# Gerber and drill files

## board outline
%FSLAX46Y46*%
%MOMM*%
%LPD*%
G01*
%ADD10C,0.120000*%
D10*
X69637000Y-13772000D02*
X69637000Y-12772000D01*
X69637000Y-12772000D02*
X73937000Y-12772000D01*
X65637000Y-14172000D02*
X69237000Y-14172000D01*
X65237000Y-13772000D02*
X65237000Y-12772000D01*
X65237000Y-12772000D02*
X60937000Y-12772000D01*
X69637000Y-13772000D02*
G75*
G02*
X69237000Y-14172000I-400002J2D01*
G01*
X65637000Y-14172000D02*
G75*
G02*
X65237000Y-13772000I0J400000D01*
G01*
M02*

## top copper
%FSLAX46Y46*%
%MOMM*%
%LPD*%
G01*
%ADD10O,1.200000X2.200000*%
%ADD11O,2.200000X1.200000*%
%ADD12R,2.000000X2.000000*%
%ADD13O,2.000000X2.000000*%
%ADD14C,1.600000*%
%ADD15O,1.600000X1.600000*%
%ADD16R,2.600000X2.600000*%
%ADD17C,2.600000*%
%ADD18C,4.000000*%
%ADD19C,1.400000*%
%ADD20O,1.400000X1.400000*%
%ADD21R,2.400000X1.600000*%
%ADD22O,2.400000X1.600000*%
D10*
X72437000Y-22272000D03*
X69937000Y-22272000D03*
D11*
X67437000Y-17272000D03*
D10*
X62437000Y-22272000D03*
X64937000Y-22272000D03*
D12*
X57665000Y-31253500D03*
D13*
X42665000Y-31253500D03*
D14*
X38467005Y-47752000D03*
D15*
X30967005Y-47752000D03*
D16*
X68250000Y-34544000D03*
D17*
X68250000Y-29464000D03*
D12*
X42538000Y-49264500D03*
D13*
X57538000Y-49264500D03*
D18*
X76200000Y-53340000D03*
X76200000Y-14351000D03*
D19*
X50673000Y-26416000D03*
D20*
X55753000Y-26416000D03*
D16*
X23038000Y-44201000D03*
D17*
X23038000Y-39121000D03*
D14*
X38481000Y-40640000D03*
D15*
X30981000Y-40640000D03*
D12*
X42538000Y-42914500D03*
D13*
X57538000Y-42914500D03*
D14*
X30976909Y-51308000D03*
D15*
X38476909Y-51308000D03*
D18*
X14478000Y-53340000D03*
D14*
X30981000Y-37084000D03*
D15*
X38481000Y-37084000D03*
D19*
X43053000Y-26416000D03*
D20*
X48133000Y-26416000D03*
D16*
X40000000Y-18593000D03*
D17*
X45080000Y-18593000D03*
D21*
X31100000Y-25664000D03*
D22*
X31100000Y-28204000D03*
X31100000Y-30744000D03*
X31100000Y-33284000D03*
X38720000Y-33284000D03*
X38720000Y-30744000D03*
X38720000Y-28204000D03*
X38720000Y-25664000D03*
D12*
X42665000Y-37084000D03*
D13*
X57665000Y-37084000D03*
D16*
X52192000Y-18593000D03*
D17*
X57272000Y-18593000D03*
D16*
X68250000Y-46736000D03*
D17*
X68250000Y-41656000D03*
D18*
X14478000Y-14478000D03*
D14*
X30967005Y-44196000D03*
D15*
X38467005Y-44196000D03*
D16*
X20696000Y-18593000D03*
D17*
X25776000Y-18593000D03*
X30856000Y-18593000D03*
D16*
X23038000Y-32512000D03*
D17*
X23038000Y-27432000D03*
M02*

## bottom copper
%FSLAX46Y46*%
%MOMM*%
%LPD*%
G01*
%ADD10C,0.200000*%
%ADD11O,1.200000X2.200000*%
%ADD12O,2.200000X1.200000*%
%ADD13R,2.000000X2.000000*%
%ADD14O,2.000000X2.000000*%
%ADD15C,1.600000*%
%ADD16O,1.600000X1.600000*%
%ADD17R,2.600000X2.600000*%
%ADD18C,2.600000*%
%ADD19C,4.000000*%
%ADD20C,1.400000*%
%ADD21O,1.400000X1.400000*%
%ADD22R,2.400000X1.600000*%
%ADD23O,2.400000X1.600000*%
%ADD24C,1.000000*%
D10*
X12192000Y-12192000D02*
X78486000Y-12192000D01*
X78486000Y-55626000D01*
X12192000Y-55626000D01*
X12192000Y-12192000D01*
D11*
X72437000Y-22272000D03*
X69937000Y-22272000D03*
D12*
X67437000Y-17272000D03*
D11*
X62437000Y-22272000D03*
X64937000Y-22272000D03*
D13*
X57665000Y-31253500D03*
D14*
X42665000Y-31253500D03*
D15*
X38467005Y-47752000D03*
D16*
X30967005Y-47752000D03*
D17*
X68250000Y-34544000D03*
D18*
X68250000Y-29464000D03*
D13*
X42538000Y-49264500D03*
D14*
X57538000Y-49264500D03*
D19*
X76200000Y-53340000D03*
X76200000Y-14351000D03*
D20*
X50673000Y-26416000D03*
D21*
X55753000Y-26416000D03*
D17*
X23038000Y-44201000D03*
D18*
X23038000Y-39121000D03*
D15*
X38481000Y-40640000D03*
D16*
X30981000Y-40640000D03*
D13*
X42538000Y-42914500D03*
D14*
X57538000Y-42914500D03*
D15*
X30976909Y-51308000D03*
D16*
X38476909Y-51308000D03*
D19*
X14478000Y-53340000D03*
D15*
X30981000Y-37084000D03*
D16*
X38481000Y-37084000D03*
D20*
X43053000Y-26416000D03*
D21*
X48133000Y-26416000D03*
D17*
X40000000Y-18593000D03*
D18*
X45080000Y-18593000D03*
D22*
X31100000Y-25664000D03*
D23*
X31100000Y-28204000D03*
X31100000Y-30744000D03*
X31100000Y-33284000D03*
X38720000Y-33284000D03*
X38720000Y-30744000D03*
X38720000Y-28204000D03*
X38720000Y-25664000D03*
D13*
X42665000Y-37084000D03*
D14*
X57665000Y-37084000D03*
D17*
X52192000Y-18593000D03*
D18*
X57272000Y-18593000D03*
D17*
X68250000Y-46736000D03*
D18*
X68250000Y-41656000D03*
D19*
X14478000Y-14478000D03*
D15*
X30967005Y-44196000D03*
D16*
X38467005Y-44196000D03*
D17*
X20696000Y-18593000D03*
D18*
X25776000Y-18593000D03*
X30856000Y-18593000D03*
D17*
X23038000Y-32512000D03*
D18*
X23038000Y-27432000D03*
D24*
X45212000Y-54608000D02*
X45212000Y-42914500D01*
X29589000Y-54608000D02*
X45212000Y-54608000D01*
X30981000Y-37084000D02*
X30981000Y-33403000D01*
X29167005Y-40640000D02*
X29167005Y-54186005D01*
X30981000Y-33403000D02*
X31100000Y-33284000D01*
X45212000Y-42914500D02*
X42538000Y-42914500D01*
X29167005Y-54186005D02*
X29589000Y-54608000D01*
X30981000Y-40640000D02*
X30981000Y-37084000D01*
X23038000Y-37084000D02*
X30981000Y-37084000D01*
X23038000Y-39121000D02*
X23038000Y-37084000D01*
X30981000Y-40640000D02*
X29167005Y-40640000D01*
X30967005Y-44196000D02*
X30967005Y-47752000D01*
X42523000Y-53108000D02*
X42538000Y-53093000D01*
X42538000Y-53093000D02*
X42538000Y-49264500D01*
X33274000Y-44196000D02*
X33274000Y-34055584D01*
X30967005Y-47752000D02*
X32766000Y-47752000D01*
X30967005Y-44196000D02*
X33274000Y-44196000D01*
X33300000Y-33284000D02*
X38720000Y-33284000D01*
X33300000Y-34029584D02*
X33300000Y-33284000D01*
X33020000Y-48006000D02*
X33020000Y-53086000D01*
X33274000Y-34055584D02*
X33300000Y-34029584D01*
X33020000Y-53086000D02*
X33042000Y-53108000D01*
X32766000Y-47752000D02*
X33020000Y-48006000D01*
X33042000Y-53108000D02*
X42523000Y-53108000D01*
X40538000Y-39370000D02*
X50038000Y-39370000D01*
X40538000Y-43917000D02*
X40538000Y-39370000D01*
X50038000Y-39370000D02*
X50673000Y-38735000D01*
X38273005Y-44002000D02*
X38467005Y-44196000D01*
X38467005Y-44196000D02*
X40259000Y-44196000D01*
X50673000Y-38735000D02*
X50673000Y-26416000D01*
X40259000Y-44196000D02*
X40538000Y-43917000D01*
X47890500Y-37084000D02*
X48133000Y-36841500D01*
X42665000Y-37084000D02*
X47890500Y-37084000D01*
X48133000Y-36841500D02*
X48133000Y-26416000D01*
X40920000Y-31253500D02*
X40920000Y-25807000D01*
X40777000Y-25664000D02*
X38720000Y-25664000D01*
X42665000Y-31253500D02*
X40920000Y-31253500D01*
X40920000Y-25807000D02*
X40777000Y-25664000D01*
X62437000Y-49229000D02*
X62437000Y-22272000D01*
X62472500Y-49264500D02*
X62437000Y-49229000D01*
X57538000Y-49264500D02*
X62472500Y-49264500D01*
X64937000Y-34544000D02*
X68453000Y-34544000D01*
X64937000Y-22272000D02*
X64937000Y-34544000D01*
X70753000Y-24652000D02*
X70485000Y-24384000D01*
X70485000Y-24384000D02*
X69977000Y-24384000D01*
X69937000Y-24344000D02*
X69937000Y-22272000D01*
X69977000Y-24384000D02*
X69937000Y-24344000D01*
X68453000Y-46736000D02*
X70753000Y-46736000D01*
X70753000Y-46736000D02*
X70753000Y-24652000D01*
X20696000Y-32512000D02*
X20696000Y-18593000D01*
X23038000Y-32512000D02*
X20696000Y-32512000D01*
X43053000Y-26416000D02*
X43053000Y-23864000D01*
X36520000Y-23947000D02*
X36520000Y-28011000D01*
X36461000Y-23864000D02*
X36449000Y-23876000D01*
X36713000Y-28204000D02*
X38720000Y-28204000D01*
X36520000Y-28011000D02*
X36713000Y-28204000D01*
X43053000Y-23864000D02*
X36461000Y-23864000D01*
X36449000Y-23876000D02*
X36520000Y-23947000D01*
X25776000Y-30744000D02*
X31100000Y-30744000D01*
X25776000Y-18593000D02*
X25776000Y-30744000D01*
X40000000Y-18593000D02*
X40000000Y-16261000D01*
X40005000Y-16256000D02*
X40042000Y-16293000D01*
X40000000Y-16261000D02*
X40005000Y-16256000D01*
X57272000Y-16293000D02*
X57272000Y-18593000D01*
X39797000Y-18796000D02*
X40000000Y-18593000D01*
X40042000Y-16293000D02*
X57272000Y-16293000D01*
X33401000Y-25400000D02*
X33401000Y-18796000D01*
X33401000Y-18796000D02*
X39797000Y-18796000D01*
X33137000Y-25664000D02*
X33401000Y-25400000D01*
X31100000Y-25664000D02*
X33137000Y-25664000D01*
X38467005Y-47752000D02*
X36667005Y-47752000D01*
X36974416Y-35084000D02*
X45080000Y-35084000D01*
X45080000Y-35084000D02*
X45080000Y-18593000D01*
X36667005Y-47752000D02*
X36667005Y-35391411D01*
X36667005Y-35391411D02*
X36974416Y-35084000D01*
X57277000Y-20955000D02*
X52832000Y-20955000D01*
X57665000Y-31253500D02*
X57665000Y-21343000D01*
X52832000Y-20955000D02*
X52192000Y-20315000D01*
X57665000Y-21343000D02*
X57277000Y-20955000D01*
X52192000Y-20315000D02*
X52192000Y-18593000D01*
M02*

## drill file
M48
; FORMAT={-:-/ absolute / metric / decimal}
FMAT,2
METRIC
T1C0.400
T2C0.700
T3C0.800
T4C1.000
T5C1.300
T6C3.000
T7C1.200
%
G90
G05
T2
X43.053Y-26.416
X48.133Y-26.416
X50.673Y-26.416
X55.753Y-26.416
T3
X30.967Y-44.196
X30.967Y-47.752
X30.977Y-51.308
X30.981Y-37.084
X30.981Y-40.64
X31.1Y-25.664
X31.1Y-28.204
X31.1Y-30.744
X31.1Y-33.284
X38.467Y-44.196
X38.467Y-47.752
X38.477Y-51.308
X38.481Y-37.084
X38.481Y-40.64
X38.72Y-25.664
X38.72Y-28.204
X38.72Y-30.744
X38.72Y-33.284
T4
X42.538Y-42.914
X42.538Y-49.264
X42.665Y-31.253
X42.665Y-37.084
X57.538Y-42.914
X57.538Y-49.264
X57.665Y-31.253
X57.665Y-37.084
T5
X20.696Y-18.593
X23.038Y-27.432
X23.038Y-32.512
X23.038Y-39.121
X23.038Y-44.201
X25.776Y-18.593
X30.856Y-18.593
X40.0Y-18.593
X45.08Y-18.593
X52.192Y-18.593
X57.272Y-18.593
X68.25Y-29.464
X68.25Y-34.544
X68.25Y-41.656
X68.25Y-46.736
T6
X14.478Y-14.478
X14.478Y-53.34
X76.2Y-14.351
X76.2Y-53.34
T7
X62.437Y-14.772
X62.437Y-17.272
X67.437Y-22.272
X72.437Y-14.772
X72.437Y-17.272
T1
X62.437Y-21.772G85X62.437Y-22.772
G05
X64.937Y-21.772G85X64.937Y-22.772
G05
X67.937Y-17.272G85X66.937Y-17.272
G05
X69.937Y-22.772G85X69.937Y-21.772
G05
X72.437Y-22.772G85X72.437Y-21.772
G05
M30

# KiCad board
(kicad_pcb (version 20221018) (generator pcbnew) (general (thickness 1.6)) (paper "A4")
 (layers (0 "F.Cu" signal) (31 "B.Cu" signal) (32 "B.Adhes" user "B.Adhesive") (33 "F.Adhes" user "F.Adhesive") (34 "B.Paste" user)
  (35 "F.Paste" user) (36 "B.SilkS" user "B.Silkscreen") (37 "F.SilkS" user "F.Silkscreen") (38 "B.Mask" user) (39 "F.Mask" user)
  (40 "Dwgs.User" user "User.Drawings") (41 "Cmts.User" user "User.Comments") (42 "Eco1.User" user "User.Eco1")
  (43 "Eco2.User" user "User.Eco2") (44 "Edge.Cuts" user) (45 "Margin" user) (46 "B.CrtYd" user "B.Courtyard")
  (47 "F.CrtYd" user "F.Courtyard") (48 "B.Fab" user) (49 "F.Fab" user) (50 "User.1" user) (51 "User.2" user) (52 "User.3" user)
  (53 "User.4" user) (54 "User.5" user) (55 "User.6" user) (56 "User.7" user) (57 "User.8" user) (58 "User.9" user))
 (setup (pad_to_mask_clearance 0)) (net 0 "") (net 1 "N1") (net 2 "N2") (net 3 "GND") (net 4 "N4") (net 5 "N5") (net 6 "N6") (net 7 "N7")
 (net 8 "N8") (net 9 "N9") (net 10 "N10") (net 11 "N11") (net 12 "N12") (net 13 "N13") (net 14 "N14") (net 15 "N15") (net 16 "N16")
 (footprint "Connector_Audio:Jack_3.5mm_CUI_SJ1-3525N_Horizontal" (layer "F.Cu") (at 67.437 17.272 180)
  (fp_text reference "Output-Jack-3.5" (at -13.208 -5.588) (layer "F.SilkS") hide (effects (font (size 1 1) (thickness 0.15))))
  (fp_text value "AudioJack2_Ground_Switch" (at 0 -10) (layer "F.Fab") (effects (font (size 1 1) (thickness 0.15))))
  (fp_line (start -2.2 3.5) (end -2.2 4.5) (stroke (width 0.12) (type solid)) (layer "Edge.Cuts"))
  (fp_line (start -2.2 4.5) (end -6.5 4.5) (stroke (width 0.12) (type solid)) (layer "Edge.Cuts"))
  (fp_line (start 1.8 3.1) (end -1.8 3.1) (stroke (width 0.12) (type solid)) (layer "Edge.Cuts"))
  (fp_line (start 2.2 3.5) (end 2.2 4.5) (stroke (width 0.12) (type solid)) (layer "Edge.Cuts"))
  (fp_line (start 2.2 4.5) (end 6.5 4.5) (stroke (width 0.12) (type solid)) (layer "Edge.Cuts"))
  (fp_arc (start -2.2 3.5) (mid -2.082842 3.217158) (end -1.8 3.1) (stroke (width 0.12) (type solid)) (layer "Edge.Cuts"))
  (fp_arc (start 1.8 3.1) (mid 2.082843 3.217157) (end 2.2 3.5) (stroke (width 0.12) (type solid)) (layer "Edge.Cuts"))
  (pad "" np_thru_hole circle (at -5 0 180) (size 1.2 1.2) (drill 1.2) (layers "*.Cu"))
  (pad "" np_thru_hole circle (at -5 2.5 180) (size 1.2 1.2) (drill 1.2) (layers "*.Cu"))
  (pad "" np_thru_hole circle (at 0 -5 180) (size 1.2 1.2) (drill 1.2) (layers "*.Cu"))
  (pad "" np_thru_hole circle (at 5 0 180) (size 1.2 1.2) (drill 1.2) (layers "*.Cu"))
  (pad "" np_thru_hole circle (at 5 2.5 180) (size 1.2 1.2) (drill 1.2) (layers "*.Cu"))
  (pad "R" thru_hole oval (at -5 -5 180) (size 1.2 2.2) (drill oval 0.4 1.4) (layers "*.Cu" "*.Mask") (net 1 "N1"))
  (pad "RN" thru_hole oval (at -2.5 -5 180) (size 1.2 2.2) (drill oval 0.4 1.4) (layers "*.Cu" "*.Mask") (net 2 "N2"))
  (pad "S" thru_hole oval (at 0 0 180) (size 2.2 1.2) (drill oval 1.4 0.4) (layers "*.Cu" "*.Mask") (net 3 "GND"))
  (pad "T" thru_hole oval (at 5 -5) (size 1.2 2.2) (drill oval 0.4 1.4) (layers "*.Cu" "*.Mask") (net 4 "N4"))
  (pad "TN" thru_hole oval (at 2.5 -5) (size 1.2 2.2) (drill oval 0.4 1.4) (layers "*.Cu" "*.Mask") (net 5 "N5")))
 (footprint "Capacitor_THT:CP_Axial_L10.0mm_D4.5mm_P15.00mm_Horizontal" (layer "F.Cu") (at 57.665 31.2535 180)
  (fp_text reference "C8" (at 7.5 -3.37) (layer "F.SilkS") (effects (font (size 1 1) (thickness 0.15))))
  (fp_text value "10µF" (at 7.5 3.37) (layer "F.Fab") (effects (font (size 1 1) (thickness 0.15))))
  (pad "1" thru_hole rect (at 0 0 180) (size 2 2) (drill 1) (layers "*.Cu" "*.Mask") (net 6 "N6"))
  (pad "2" thru_hole oval (at 15 0 180) (size 2 2) (drill 1) (layers "*.Cu" "*.Mask") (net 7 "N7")))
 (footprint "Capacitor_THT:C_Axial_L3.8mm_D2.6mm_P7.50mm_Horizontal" (layer "F.Cu") (at 38.467005 47.752 180)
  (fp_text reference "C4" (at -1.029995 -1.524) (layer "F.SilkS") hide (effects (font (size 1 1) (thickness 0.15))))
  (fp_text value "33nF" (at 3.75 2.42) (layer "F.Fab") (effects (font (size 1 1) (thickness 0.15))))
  (pad "1" thru_hole circle (at 0 0 180) (size 1.6 1.6) (drill 0.8) (layers "*.Cu" "*.Mask") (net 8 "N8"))
  (pad "2" thru_hole oval (at 7.5 0 180) (size 1.6 1.6) (drill 0.8) (layers "*.Cu" "*.Mask") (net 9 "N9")))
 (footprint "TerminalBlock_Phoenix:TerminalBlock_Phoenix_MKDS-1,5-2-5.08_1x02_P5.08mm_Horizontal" (layer "F.Cu") (at 68.25 34.544 90)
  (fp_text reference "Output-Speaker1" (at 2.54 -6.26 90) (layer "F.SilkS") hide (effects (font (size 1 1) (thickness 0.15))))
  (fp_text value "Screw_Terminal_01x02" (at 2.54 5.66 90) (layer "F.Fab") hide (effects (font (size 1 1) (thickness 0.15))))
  (pad "1" thru_hole rect (at 0 0 90) (size 2.6 2.6) (drill 1.3) (layers "*.Cu" "*.Mask") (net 5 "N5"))
  (pad "2" thru_hole circle (at 5.08 0 90) (size 2.6 2.6) (drill 1.3) (layers "*.Cu" "*.Mask") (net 3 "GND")))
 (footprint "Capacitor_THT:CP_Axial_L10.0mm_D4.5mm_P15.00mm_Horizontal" (layer "F.Cu") (at 42.538 49.2645)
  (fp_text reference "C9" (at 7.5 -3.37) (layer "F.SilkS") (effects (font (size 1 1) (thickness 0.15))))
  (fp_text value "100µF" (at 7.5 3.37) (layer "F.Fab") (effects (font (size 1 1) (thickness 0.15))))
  (pad "1" thru_hole rect (at 0 0) (size 2 2) (drill 1) (layers "*.Cu" "*.Mask") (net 9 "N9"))
  (pad "2" thru_hole oval (at 15 0) (size 2 2) (drill 1) (layers "*.Cu" "*.Mask") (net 4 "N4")))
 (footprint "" (layer "F.Cu") (at 76.2 53.34)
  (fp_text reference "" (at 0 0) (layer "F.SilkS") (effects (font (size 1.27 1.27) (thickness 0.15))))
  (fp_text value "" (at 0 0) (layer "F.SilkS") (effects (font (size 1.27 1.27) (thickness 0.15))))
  (pad "" thru_hole circle (at 0 0) (size 4 4) (drill 3) (layers "*.Cu" "*.Mask") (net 3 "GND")))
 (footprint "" (layer "F.Cu") (at 76.2 14.351)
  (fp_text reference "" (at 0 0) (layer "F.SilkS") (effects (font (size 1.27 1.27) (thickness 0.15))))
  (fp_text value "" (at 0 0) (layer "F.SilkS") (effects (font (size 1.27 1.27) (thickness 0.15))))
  (pad "" thru_hole circle (at 0 0) (size 4 4) (drill 3) (layers "*.Cu" "*.Mask") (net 3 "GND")))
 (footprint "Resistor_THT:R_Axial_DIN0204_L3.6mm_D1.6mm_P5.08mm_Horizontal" (layer "F.Cu") (at 50.673 26.416)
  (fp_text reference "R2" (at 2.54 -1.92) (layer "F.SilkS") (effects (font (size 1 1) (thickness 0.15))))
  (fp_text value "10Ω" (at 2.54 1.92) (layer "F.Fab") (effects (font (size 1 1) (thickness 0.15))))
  (pad "1" thru_hole circle (at 0 0) (size 1.4 1.4) (drill 0.7) (layers "*.Cu" "*.Mask") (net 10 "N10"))
  (pad "2" thru_hole oval (at 5.08 0) (size 1.4 1.4) (drill 0.7) (layers "*.Cu" "*.Mask") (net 3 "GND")))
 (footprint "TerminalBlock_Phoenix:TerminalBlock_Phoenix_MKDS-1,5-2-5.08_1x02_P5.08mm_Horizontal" (layer "F.Cu") (at 23.038 44.201 90)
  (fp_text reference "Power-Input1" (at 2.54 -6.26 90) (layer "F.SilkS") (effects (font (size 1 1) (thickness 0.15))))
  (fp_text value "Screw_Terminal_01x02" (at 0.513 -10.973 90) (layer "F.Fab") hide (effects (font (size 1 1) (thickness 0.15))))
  (pad "1" thru_hole rect (at 0 0 90) (size 2.6 2.6) (drill 1.3) (layers "*.Cu" "*.Mask") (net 3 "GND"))
  (pad "2" thru_hole circle (at 5.08 0 90) (size 2.6 2.6) (drill 1.3) (layers "*.Cu" "*.Mask") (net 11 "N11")))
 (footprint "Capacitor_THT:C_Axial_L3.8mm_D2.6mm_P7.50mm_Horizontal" (layer "F.Cu") (at 38.481 40.64 180)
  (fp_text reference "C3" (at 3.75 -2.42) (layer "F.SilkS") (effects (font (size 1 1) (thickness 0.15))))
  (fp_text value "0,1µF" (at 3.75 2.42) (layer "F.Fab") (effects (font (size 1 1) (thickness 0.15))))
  (pad "1" thru_hole circle (at 0 0 180) (size 1.6 1.6) (drill 0.8) (layers "*.Cu" "*.Mask") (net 3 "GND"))
  (pad "2" thru_hole oval (at 7.5 0 180) (size 1.6 1.6) (drill 0.8) (layers "*.Cu" "*.Mask") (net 11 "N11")))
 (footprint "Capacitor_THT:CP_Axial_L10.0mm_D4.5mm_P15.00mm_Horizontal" (layer "F.Cu") (at 42.538 42.9145)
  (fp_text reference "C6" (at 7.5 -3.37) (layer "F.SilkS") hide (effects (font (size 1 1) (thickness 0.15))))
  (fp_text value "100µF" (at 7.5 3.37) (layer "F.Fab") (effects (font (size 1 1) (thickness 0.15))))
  (pad "1" thru_hole rect (at 0 0) (size 2 2) (drill 1) (layers "*.Cu" "*.Mask") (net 11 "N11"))
  (pad "2" thru_hole oval (at 15 0) (size 2 2) (drill 1) (layers "*.Cu" "*.Mask") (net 3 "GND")))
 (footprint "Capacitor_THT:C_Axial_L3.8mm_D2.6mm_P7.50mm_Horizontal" (layer "F.Cu") (at 30.976909 51.308)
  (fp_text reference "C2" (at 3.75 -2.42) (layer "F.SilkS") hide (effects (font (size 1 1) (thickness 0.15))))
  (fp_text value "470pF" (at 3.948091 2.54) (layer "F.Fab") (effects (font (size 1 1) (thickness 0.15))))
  (pad "1" thru_hole circle (at 0 0) (size 1.6 1.6) (drill 0.8) (layers "*.Cu" "*.Mask") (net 3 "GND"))
  (pad "2" thru_hole oval (at 7.5 0) (size 1.6 1.6) (drill 0.8) (layers "*.Cu" "*.Mask") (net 3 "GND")))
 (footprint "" (layer "F.Cu") (at 14.478 53.34)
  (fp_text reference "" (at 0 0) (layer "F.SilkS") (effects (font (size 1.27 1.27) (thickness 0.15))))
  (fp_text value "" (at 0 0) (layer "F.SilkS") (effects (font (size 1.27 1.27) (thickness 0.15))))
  (pad "" thru_hole circle (at 0 0) (size 4 4) (drill 3) (layers "*.Cu" "*.Mask") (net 3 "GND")))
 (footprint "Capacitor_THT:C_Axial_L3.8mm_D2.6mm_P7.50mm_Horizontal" (layer "F.Cu") (at 30.981 37.084)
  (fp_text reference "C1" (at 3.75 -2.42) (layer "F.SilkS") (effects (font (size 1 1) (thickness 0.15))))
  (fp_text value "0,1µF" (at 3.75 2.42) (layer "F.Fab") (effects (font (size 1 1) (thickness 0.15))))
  (pad "1" thru_hole circle (at 0 0) (size 1.6 1.6) (drill 0.8) (layers "*.Cu" "*.Mask") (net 11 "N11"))
  (pad "2" thru_hole oval (at 7.5 0) (size 1.6 1.6) (drill 0.8) (layers "*.Cu" "*.Mask") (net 3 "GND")))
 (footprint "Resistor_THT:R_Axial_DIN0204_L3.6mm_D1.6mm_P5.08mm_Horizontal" (layer "F.Cu") (at 43.053 26.416)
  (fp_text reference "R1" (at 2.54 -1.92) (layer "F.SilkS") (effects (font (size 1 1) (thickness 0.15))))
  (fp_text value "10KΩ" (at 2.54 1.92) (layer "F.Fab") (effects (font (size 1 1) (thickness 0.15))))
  (pad "1" thru_hole circle (at 0 0) (size 1.4 1.4) (drill 0.7) (layers "*.Cu" "*.Mask") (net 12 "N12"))
  (pad "2" thru_hole oval (at 5.08 0) (size 1.4 1.4) (drill 0.7) (layers "*.Cu" "*.Mask") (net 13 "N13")))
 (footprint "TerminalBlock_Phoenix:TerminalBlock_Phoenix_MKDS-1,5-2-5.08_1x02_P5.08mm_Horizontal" (layer "F.Cu") (at 40 18.593)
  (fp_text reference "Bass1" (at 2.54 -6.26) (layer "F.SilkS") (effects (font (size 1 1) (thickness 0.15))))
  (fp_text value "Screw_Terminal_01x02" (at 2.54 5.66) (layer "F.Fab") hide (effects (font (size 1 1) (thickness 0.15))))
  (pad "1" thru_hole rect (at 0 0) (size 2.6 2.6) (drill 1.3) (layers "*.Cu" "*.Mask") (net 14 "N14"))
  (pad "2" thru_hole circle (at 5.08 0) (size 2.6 2.6) (drill 1.3) (layers "*.Cu" "*.Mask") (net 8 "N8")))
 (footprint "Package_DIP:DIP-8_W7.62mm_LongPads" (layer "F.Cu") (at 31.1 25.664)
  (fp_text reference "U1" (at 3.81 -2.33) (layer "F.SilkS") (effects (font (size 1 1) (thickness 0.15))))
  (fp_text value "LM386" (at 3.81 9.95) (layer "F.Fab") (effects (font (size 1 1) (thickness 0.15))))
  (pad "1" thru_hole rect (at 0 0) (size 2.4 1.6) (drill 0.8) (layers "*.Cu" "*.Mask") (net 14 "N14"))
  (pad "2" thru_hole oval (at 0 2.54) (size 2.4 1.6) (drill 0.8) (layers "*.Cu" "*.Mask") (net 3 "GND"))
  (pad "3" thru_hole oval (at 0 5.08) (size 2.4 1.6) (drill 0.8) (layers "*.Cu" "*.Mask") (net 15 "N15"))
  (pad "4" thru_hole oval (at 0 7.62) (size 2.4 1.6) (drill 0.8) (layers "*.Cu" "*.Mask") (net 11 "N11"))
  (pad "5" thru_hole oval (at 7.62 7.62) (size 2.4 1.6) (drill 0.8) (layers "*.Cu" "*.Mask") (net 9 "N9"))
  (pad "6" thru_hole oval (at 7.62 5.08) (size 2.4 1.6) (drill 0.8) (layers "*.Cu" "*.Mask") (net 3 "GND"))
  (pad "7" thru_hole oval (at 7.62 2.54) (size 2.4 1.6) (drill 0.8) (layers "*.Cu" "*.Mask") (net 12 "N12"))
  (pad "8" thru_hole oval (at 7.62 0) (size 2.4 1.6) (drill 0.8) (layers "*.Cu" "*.Mask") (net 7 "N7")))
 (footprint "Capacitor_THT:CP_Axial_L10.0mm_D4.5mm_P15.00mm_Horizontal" (layer "F.Cu") (at 42.665 37.084)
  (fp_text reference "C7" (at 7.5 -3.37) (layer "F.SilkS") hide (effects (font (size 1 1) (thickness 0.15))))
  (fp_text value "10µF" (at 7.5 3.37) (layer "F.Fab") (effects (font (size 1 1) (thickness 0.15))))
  (pad "1" thru_hole rect (at 0 0) (size 2 2) (drill 1) (layers "*.Cu" "*.Mask") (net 13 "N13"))
  (pad "2" thru_hole oval (at 15 0) (size 2 2) (drill 1) (layers "*.Cu" "*.Mask") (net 3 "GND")))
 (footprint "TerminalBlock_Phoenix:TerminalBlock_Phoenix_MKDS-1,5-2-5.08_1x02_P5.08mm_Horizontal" (layer "F.Cu") (at 52.192 18.593)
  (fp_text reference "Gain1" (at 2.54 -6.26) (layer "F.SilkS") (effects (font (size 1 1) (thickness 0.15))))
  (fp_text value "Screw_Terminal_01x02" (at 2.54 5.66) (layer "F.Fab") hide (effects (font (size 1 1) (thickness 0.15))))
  (pad "1" thru_hole rect (at 0 0) (size 2.6 2.6) (drill 1.3) (layers "*.Cu" "*.Mask") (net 6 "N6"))
  (pad "2" thru_hole circle (at 5.08 0) (size 2.6 2.6) (drill 1.3) (layers "*.Cu" "*.Mask") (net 14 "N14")))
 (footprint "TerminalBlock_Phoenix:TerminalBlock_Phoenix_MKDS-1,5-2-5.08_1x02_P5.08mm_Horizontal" (layer "F.Cu") (at 68.25 46.736 90)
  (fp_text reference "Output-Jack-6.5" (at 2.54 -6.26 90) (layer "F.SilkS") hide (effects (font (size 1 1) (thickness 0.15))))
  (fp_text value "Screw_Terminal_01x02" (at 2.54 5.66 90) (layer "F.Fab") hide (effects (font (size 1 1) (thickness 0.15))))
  (pad "1" thru_hole rect (at 0 0 90) (size 2.6 2.6) (drill 1.3) (layers "*.Cu" "*.Mask") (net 2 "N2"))
  (pad "2" thru_hole circle (at 5.08 0 90) (size 2.6 2.6) (drill 1.3) (layers "*.Cu" "*.Mask") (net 3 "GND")))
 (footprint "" (layer "F.Cu") (at 14.478 14.478)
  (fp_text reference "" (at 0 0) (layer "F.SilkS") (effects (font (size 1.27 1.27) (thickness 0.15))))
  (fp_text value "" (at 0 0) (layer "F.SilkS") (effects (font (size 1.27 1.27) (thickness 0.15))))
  (pad "" thru_hole circle (at 0 0) (size 4 4) (drill 3) (layers "*.Cu" "*.Mask") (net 3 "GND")))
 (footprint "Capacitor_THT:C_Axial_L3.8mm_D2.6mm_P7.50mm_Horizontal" (layer "F.Cu") (at 30.967005 44.196)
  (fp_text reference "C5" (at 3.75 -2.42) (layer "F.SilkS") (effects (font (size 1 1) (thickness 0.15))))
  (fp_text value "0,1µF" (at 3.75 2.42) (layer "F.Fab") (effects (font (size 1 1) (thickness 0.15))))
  (pad "1" thru_hole circle (at 0 0) (size 1.6 1.6) (drill 0.8) (layers "*.Cu" "*.Mask") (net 9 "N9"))
  (pad "2" thru_hole oval (at 7.5 0) (size 1.6 1.6) (drill 0.8) (layers "*.Cu" "*.Mask") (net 10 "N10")))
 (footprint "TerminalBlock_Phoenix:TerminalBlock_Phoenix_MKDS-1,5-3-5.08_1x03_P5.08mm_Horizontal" (layer "F.Cu") (at 20.696 18.593)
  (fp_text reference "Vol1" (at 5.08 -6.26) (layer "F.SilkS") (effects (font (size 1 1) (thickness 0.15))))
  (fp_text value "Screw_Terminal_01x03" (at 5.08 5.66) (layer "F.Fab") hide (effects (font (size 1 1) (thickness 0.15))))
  (pad "1" thru_hole rect (at 0 0) (size 2.6 2.6) (drill 1.3) (layers "*.Cu" "*.Mask") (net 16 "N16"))
  (pad "2" thru_hole circle (at 5.08 0) (size 2.6 2.6) (drill 1.3) (layers "*.Cu" "*.Mask") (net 15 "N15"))
  (pad "3" thru_hole circle (at 10.16 0) (size 2.6 2.6) (drill 1.3) (layers "*.Cu" "*.Mask") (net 3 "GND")))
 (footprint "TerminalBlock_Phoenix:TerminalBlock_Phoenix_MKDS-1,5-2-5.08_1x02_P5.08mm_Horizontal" (layer "F.Cu") (at 23.038 32.512 90)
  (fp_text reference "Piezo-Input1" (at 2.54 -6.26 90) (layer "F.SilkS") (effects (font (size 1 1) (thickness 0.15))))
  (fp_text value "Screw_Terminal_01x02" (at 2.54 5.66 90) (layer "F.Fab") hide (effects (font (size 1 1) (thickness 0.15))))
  (pad "1" thru_hole rect (at 0 0 90) (size 2.6 2.6) (drill 1.3) (layers "*.Cu" "*.Mask") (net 16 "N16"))
  (pad "2" thru_hole circle (at 5.08 0 90) (size 2.6 2.6) (drill 1.3) (layers "*.Cu" "*.Mask") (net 3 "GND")))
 (gr_rect (start 12.192 12.192) (end 78.486 55.626) (stroke (width 0.2) (type default)) (fill none) (layer "B.Cu"))
 (segment (start 45.212 54.608) (end 45.212 42.9145) (width 1) (layer "B.Cu") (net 11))
 (segment (start 29.589 54.608) (end 45.212 54.608) (width 1) (layer "B.Cu") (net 11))
 (segment (start 30.981 37.084) (end 30.981 33.403) (width 1) (layer "B.Cu") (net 11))
 (segment (start 29.167005 40.64) (end 29.167005 54.186005) (width 1) (layer "B.Cu") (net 11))
 (segment (start 30.981 33.403) (end 31.1 33.284) (width 1) (layer "B.Cu") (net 11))
 (segment (start 45.212 42.9145) (end 42.538 42.9145) (width 1) (layer "B.Cu") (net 11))
 (segment (start 29.167005 54.186005) (end 29.589 54.608) (width 1) (layer "B.Cu") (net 11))
 (segment (start 30.981 40.64) (end 30.981 37.084) (width 1) (layer "B.Cu") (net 11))
 (segment (start 23.038 37.084) (end 30.981 37.084) (width 1) (layer "B.Cu") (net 11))
 (segment (start 23.038 39.121) (end 23.038 37.084) (width 1) (layer "B.Cu") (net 11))
 (segment (start 30.981 40.64) (end 29.167005 40.64) (width 1) (layer "B.Cu") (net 11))
 (segment (start 30.967005 44.196) (end 30.967005 47.752) (width 1) (layer "B.Cu") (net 9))
 (segment (start 42.523 53.108) (end 42.538 53.093) (width 1) (layer "B.Cu") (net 9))
 (segment (start 42.538 53.093) (end 42.538 49.2645) (width 1) (layer "B.Cu") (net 9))
 (segment (start 33.274 44.196) (end 33.274 34.055584) (width 1) (layer "B.Cu") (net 9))
 (segment (start 30.967005 47.752) (end 32.766 47.752) (width 1) (layer "B.Cu") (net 9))
 (segment (start 30.967005 44.196) (end 33.274 44.196) (width 1) (layer "B.Cu") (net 9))
 (segment (start 33.3 33.284) (end 38.72 33.284) (width 1) (layer "B.Cu") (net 9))
 (segment (start 33.3 34.029584) (end 33.3 33.284) (width 1) (layer "B.Cu") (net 9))
 (segment (start 33.02 48.006) (end 33.02 53.086) (width 1) (layer "B.Cu") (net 9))
 (segment (start 33.274 34.055584) (end 33.3 34.029584) (width 1) (layer "B.Cu") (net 9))
 (segment (start 33.02 53.086) (end 33.042 53.108) (width 1) (layer "B.Cu") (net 9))
 (segment (start 32.766 47.752) (end 33.02 48.006) (width 1) (layer "B.Cu") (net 9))
 (segment (start 33.042 53.108) (end 42.523 53.108) (width 1) (layer "B.Cu") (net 9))
 (segment (start 40.538 39.37) (end 50.038 39.37) (width 1) (layer "B.Cu") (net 10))
 (segment (start 40.538 43.917) (end 40.538 39.37) (width 1) (layer "B.Cu") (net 10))
 (segment (start 50.038 39.37) (end 50.673 38.735) (width 1) (layer "B.Cu") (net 10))
 (segment (start 38.273005 44.002) (end 38.467005 44.196) (width 1) (layer "B.Cu") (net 10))
 (segment (start 38.467005 44.196) (end 40.259 44.196) (width 1) (layer "B.Cu") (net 10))
 (segment (start 50.673 38.735) (end 50.673 26.416) (width 1) (layer "B.Cu") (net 10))
 (segment (start 40.259 44.196) (end 40.538 43.917) (width 1) (layer "B.Cu") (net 10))
 (segment (start 47.8905 37.084) (end 48.133 36.8415) (width 1) (layer "B.Cu") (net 13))
 (segment (start 42.665 37.084) (end 47.8905 37.084) (width 1) (layer "B.Cu") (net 13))
 (segment (start 48.133 36.8415) (end 48.133 26.416) (width 1) (layer "B.Cu") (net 13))
 (segment (start 40.92 31.2535) (end 40.92 25.807) (width 1) (layer "B.Cu") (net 7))
 (segment (start 40.777 25.664) (end 38.72 25.664) (width 1) (layer "B.Cu") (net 7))
 (segment (start 42.665 31.2535) (end 40.92 31.2535) (width 1) (layer "B.Cu") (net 7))
 (segment (start 40.92 25.807) (end 40.777 25.664) (width 1) (layer "B.Cu") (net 7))
 (segment (start 62.437 49.229) (end 62.437 22.272) (width 1) (layer "B.Cu") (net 4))
 (segment (start 62.4725 49.2645) (end 62.437 49.229) (width 1) (layer "B.Cu") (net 4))
 (segment (start 57.538 49.2645) (end 62.4725 49.2645) (width 1) (layer "B.Cu") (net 4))
 (segment (start 64.937 34.544) (end 68.453 34.544) (width 1) (layer "B.Cu") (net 5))
 (segment (start 64.937 22.272) (end 64.937 34.544) (width 1) (layer "B.Cu") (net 5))
 (segment (start 70.753 24.652) (end 70.485 24.384) (width 1) (layer "B.Cu") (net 2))
 (segment (start 70.485 24.384) (end 69.977 24.384) (width 1) (layer "B.Cu") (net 2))
 (segment (start 69.937 24.344) (end 69.937 22.272) (width 1) (layer "B.Cu") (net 2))
 (segment (start 69.977 24.384) (end 69.937 24.344) (width 1) (layer "B.Cu") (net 2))
 (segment (start 68.453 46.736) (end 70.753 46.736) (width 1) (layer "B.Cu") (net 2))
 (segment (start 70.753 46.736) (end 70.753 24.652) (width 1) (layer "B.Cu") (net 2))
 (segment (start 20.696 32.512) (end 20.696 18.593) (width 1) (layer "B.Cu") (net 16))
 (segment (start 23.038 32.512) (end 20.696 32.512) (width 1) (layer "B.Cu") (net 16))
 (segment (start 43.053 26.416) (end 43.053 23.864) (width 1) (layer "B.Cu") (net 12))
 (segment (start 36.52 23.947) (end 36.52 28.011) (width 1) (layer "B.Cu") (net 12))
 (segment (start 36.461 23.864) (end 36.449 23.876) (width 1) (layer "B.Cu") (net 12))
 (segment (start 36.713 28.204) (end 38.72 28.204) (width 1) (layer "B.Cu") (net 12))
 (segment (start 36.52 28.011) (end 36.713 28.204) (width 1) (layer "B.Cu") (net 12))
 (segment (start 43.053 23.864) (end 36.461 23.864) (width 1) (layer "B.Cu") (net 12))
 (segment (start 36.449 23.876) (end 36.52 23.947) (width 1) (layer "B.Cu") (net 12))
 (segment (start 25.776 30.744) (end 31.1 30.744) (width 1) (layer "B.Cu") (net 15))
 (segment (start 25.776 18.593) (end 25.776 30.744) (width 1) (layer "B.Cu") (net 15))
 (segment (start 40 18.593) (end 40 16.261) (width 1) (layer "B.Cu") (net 14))
 (segment (start 40.005 16.256) (end 40.042 16.293) (width 1) (layer "B.Cu") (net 14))
 (segment (start 40 16.261) (end 40.005 16.256) (width 1) (layer "B.Cu") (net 14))
 (segment (start 57.272 16.293) (end 57.272 18.593) (width 1) (layer "B.Cu") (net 14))
 (segment (start 39.797 18.796) (end 40 18.593) (width 1) (layer "B.Cu") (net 14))
 (segment (start 40.042 16.293) (end 57.272 16.293) (width 1) (layer "B.Cu") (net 14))
 (segment (start 33.401 25.4) (end 33.401 18.796) (width 1) (layer "B.Cu") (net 14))
 (segment (start 33.401 18.796) (end 39.797 18.796) (width 1) (layer "B.Cu") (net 14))
 (segment (start 33.137 25.664) (end 33.401 25.4) (width 1) (layer "B.Cu") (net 14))
 (segment (start 31.1 25.664) (end 33.137 25.664) (width 1) (layer "B.Cu") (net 14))
 (segment (start 38.467005 47.752) (end 36.667005 47.752) (width 1) (layer "B.Cu") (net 8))
 (segment (start 36.974416 35.084) (end 45.08 35.084) (width 1) (layer "B.Cu") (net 8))
 (segment (start 45.08 35.084) (end 45.08 18.593) (width 1) (layer "B.Cu") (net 8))
 (segment (start 36.667005 47.752) (end 36.667005 35.391411) (width 1) (layer "B.Cu") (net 8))
 (segment (start 36.667005 35.391411) (end 36.974416 35.084) (width 1) (layer "B.Cu") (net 8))
 (segment (start 57.277 20.955) (end 52.832 20.955) (width 1) (layer "B.Cu") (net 6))
 (segment (start 57.665 31.2535) (end 57.665 21.343) (width 1) (layer "B.Cu") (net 6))
 (segment (start 52.832 20.955) (end 52.192 20.315) (width 1) (layer "B.Cu") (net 6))
 (segment (start 57.665 21.343) (end 57.277 20.955) (width 1) (layer "B.Cu") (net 6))
 (segment (start 52.192 20.315) (end 52.192 18.593) (width 1) (layer "B.Cu") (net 6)))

